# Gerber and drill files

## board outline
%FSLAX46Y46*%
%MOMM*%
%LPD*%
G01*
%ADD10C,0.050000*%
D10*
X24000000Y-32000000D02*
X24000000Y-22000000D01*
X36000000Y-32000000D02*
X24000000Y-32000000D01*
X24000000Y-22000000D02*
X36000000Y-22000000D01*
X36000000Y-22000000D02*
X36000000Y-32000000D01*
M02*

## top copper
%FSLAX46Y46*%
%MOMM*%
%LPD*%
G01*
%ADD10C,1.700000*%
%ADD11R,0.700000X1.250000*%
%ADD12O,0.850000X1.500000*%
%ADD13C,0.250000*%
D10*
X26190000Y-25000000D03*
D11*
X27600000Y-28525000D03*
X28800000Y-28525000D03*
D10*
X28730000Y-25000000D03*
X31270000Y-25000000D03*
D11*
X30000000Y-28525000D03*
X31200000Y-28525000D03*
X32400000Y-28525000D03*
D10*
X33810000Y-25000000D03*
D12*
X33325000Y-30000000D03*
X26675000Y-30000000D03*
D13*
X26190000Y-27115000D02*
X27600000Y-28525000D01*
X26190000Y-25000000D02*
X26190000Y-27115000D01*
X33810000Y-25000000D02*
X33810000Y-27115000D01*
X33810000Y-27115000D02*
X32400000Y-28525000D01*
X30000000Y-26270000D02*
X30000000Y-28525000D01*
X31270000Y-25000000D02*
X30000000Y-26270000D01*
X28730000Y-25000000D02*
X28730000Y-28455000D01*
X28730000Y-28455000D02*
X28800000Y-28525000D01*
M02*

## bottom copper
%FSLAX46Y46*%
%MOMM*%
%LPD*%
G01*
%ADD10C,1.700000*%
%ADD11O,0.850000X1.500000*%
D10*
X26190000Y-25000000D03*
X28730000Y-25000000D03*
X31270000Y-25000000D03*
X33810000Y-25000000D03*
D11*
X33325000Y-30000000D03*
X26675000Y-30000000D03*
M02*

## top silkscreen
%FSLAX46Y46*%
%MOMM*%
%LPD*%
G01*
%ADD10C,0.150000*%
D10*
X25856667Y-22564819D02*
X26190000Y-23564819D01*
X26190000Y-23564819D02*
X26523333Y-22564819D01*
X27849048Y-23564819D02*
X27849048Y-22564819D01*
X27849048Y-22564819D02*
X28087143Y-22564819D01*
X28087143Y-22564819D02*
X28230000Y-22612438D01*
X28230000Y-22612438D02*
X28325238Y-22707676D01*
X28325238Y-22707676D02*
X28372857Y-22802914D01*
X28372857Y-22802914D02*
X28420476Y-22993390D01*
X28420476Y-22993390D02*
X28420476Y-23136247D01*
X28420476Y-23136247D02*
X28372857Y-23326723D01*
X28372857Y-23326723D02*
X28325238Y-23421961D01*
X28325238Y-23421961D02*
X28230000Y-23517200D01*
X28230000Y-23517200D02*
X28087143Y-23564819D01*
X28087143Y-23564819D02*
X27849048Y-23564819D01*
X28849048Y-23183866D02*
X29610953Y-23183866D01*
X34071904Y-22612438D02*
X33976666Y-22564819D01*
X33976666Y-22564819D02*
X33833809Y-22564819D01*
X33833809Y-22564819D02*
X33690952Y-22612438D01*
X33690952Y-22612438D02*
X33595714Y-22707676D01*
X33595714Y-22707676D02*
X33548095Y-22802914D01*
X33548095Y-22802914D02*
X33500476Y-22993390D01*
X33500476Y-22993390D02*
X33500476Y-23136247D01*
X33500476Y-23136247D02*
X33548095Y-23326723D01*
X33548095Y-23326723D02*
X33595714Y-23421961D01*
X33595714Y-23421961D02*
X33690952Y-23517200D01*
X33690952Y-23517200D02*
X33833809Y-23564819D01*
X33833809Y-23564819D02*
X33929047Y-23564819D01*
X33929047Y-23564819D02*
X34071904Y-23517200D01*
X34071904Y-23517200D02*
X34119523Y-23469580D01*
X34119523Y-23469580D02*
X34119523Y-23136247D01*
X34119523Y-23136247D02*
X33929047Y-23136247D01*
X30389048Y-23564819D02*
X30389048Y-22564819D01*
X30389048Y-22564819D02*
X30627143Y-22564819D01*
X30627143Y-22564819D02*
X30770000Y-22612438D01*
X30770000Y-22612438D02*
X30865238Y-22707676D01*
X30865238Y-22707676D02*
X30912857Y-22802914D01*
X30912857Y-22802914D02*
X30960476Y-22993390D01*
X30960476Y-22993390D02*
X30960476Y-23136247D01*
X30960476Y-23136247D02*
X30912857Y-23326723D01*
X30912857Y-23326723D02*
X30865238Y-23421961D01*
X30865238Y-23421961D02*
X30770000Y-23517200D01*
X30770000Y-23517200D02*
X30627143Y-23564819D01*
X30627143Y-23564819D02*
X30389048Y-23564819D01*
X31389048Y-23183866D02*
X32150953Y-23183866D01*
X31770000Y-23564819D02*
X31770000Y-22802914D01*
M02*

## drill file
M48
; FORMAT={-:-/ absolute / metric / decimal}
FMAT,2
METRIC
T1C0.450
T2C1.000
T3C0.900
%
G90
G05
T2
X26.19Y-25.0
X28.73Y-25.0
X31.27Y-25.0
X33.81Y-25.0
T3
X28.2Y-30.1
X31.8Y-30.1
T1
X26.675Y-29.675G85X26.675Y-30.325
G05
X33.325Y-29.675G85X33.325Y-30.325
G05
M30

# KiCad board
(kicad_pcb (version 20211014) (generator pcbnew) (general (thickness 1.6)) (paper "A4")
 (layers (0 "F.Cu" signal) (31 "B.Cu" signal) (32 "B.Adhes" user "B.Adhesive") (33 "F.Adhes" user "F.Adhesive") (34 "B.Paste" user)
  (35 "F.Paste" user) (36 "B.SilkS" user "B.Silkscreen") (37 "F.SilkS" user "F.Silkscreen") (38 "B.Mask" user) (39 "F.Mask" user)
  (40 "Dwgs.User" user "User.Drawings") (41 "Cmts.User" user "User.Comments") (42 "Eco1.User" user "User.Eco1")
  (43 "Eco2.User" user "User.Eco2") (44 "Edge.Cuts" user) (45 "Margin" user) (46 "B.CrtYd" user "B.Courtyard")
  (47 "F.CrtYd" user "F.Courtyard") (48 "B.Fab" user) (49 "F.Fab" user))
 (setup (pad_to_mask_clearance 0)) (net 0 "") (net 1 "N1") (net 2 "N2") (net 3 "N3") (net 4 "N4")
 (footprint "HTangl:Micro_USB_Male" (layer "F.Cu") (at 30 30)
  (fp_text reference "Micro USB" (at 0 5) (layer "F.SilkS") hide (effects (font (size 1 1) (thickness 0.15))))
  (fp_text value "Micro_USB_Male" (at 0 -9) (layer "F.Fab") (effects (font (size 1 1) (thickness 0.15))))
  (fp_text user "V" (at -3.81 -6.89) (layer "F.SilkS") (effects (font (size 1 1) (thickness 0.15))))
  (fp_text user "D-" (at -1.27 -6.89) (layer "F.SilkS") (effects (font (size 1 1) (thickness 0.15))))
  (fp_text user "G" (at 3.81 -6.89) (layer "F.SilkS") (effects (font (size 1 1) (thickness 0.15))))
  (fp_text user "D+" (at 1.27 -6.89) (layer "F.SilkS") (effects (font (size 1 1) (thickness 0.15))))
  (pad "" np_thru_hole circle (at -1.8 0.1) (size 0.9 0.9) (drill 0.9) (layers *.Cu *.Mask))
  (pad "" np_thru_hole circle (at 1.8 0.1) (size 0.9 0.9) (drill 0.9) (layers *.Cu *.Mask))
  (pad "1" thru_hole circle (at -3.81 -5) (size 1.7 1.7) (drill 1) (layers *.Cu *.Mask) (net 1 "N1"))
  (pad "1" smd rect (at -2.4 -1.475) (size 0.7 1.25) (layers "F.Cu" "F.Paste" "F.Mask") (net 1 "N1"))
  (pad "2" smd rect (at -1.2 -1.475) (size 0.7 1.25) (layers "F.Cu" "F.Paste" "F.Mask") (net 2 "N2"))
  (pad "2" thru_hole circle (at -1.27 -5) (size 1.7 1.7) (drill 1) (layers *.Cu *.Mask) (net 2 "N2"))
  (pad "3" thru_hole circle (at 1.27 -5) (size 1.7 1.7) (drill 1) (layers *.Cu *.Mask) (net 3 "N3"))
  (pad "3" smd rect (at 0 -1.475) (size 0.7 1.25) (layers "F.Cu" "F.Paste" "F.Mask") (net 3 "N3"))
  (pad "4" smd rect (at 1.2 -1.475) (size 0.7 1.25) (layers "F.Cu" "F.Paste" "F.Mask"))
  (pad "5" smd rect (at 2.4 -1.475) (size 0.7 1.25) (layers "F.Cu" "F.Paste" "F.Mask") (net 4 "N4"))
  (pad "5" thru_hole circle (at 3.81 -5) (size 1.7 1.7) (drill 1) (layers *.Cu *.Mask) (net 4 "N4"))
  (pad "6" thru_hole oval (at 3.325 0) (size 0.85 1.5) (drill oval 0.45 1.1) (layers *.Cu *.Mask))
  (pad "6" thru_hole oval (at -3.325 0) (size 0.85 1.5) (drill oval 0.45 1.1) (layers *.Cu *.Mask)))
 (gr_line (start 24 32) (end 24 22) (layer "Edge.Cuts") (width 0.05))
 (gr_line (start 36 32) (end 24 32) (layer "Edge.Cuts") (width 0.05))
 (gr_line (start 24 22) (end 36 22) (layer "Edge.Cuts") (width 0.05))
 (gr_line (start 36 22) (end 36 32) (layer "Edge.Cuts") (width 0.05))
 (segment (start 26.19 27.115) (end 27.6 28.525) (width 0.25) (layer "F.Cu") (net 1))
 (segment (start 26.19 25) (end 26.19 27.115) (width 0.25) (layer "F.Cu") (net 1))
 (segment (start 33.81 25) (end 33.81 27.115) (width 0.25) (layer "F.Cu") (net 4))
 (segment (start 33.81 27.115) (end 32.4 28.525) (width 0.25) (layer "F.Cu") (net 4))
 (segment (start 30 26.27) (end 30 28.525) (width 0.25) (layer "F.Cu") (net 3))
 (segment (start 31.27 25) (end 30 26.27) (width 0.25) (layer "F.Cu") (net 3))
 (segment (start 28.73 25) (end 28.73 28.455) (width 0.25) (layer "F.Cu") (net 2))
 (segment (start 28.73 28.455) (end 28.8 28.525) (width 0.25) (layer "F.Cu") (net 2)))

